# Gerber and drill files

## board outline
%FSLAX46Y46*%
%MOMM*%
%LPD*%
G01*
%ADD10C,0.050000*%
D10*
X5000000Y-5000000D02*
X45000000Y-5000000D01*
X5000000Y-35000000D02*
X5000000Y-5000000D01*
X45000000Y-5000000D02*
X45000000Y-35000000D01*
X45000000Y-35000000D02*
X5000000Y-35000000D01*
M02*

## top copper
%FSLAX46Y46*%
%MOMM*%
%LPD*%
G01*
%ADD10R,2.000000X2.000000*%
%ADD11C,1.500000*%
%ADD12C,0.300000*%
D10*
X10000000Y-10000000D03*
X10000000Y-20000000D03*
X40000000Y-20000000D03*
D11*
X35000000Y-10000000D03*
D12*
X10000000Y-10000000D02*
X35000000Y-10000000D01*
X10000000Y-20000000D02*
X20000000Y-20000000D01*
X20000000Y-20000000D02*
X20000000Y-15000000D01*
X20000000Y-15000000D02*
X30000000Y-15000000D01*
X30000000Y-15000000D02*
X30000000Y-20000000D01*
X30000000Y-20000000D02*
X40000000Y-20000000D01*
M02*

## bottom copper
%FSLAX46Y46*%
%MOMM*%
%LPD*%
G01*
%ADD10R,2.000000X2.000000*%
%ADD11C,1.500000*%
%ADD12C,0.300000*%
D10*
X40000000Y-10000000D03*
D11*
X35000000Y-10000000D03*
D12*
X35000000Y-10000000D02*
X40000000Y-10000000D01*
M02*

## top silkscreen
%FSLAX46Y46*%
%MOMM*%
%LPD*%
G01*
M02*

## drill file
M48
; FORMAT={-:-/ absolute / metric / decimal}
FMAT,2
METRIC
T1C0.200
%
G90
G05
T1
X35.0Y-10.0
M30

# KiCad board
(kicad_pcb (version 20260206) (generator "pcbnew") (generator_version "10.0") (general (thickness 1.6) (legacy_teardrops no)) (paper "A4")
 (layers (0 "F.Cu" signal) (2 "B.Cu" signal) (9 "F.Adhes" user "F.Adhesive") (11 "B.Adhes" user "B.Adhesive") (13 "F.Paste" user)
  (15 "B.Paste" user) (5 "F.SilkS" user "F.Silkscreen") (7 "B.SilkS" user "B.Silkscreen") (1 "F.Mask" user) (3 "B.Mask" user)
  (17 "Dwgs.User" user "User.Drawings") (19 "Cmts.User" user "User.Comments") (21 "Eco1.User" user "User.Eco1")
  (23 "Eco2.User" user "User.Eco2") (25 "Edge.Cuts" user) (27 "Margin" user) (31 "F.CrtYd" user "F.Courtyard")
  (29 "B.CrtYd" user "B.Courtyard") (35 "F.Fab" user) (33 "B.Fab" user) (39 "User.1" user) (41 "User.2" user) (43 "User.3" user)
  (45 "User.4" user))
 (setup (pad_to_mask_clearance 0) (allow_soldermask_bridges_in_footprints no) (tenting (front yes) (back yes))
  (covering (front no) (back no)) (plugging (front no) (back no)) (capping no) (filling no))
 (gr_line (start 5 5) (end 45 5) (stroke (width 0.05) (type default)) (layer "Edge.Cuts"))
 (gr_line (start 5 35) (end 5 5) (stroke (width 0.05) (type default)) (layer "Edge.Cuts"))
 (gr_line (start 45 5) (end 45 35) (stroke (width 0.05) (type default)) (layer "Edge.Cuts"))
 (gr_line (start 45 35) (end 5 35) (stroke (width 0.05) (type default)) (layer "Edge.Cuts"))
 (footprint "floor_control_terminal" (layer "F.Cu") (at 10 10)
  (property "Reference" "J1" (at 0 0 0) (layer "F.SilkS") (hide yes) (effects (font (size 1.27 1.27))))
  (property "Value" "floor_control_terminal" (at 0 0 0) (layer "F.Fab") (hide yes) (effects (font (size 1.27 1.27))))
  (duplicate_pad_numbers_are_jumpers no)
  (pad "1" smd rect (at 0 0) (size 2 2) (layers "F.Cu" "F.Paste" "F.Mask") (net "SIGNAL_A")))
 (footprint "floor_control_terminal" (layer "B.Cu") (at 40 10)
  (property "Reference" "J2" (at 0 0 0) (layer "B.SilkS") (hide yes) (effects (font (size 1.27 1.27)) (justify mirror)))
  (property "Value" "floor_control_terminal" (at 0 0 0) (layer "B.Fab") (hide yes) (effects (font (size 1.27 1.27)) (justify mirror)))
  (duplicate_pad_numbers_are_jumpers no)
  (pad "1" smd rect (at 0 0) (size 2 2) (layers "B.Cu" "B.Paste" "B.Mask") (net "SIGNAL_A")))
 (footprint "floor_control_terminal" (layer "F.Cu") (at 10 20)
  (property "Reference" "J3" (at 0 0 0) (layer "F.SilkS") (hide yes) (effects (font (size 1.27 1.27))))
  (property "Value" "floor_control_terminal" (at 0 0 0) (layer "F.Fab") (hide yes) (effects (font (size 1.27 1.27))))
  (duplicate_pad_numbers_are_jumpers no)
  (pad "1" smd rect (at 0 0) (size 2 2) (layers "F.Cu" "F.Paste" "F.Mask") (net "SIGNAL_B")))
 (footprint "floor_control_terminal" (layer "F.Cu") (at 40 20)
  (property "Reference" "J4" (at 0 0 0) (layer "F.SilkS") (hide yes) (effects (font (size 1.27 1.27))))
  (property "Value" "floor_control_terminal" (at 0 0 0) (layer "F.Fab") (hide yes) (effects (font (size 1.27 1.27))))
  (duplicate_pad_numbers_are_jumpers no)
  (pad "1" smd rect (at 0 0) (size 2 2) (layers "F.Cu" "F.Paste" "F.Mask") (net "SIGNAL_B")))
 (segment (start 10 10) (end 35 10) (width 0.3) (layer "F.Cu") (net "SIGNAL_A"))
 (segment (start 35 10) (end 40 10) (width 0.3) (layer "B.Cu") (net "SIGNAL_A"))
 (via (at 35 10) (size 1.5) (drill 0.2) (layers "F.Cu" "B.Cu") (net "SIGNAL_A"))
 (segment (start 10 20) (end 20 20) (width 0.3) (layer "F.Cu") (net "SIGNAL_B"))
 (segment (start 20 20) (end 20 15) (width 0.3) (layer "F.Cu") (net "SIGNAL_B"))
 (segment (start 20 15) (end 30 15) (width 0.3) (layer "F.Cu") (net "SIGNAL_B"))
 (segment (start 30 15) (end 30 20) (width 0.3) (layer "F.Cu") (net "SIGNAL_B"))
 (segment (start 30 20) (end 40 20) (width 0.3) (layer "F.Cu") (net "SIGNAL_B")))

